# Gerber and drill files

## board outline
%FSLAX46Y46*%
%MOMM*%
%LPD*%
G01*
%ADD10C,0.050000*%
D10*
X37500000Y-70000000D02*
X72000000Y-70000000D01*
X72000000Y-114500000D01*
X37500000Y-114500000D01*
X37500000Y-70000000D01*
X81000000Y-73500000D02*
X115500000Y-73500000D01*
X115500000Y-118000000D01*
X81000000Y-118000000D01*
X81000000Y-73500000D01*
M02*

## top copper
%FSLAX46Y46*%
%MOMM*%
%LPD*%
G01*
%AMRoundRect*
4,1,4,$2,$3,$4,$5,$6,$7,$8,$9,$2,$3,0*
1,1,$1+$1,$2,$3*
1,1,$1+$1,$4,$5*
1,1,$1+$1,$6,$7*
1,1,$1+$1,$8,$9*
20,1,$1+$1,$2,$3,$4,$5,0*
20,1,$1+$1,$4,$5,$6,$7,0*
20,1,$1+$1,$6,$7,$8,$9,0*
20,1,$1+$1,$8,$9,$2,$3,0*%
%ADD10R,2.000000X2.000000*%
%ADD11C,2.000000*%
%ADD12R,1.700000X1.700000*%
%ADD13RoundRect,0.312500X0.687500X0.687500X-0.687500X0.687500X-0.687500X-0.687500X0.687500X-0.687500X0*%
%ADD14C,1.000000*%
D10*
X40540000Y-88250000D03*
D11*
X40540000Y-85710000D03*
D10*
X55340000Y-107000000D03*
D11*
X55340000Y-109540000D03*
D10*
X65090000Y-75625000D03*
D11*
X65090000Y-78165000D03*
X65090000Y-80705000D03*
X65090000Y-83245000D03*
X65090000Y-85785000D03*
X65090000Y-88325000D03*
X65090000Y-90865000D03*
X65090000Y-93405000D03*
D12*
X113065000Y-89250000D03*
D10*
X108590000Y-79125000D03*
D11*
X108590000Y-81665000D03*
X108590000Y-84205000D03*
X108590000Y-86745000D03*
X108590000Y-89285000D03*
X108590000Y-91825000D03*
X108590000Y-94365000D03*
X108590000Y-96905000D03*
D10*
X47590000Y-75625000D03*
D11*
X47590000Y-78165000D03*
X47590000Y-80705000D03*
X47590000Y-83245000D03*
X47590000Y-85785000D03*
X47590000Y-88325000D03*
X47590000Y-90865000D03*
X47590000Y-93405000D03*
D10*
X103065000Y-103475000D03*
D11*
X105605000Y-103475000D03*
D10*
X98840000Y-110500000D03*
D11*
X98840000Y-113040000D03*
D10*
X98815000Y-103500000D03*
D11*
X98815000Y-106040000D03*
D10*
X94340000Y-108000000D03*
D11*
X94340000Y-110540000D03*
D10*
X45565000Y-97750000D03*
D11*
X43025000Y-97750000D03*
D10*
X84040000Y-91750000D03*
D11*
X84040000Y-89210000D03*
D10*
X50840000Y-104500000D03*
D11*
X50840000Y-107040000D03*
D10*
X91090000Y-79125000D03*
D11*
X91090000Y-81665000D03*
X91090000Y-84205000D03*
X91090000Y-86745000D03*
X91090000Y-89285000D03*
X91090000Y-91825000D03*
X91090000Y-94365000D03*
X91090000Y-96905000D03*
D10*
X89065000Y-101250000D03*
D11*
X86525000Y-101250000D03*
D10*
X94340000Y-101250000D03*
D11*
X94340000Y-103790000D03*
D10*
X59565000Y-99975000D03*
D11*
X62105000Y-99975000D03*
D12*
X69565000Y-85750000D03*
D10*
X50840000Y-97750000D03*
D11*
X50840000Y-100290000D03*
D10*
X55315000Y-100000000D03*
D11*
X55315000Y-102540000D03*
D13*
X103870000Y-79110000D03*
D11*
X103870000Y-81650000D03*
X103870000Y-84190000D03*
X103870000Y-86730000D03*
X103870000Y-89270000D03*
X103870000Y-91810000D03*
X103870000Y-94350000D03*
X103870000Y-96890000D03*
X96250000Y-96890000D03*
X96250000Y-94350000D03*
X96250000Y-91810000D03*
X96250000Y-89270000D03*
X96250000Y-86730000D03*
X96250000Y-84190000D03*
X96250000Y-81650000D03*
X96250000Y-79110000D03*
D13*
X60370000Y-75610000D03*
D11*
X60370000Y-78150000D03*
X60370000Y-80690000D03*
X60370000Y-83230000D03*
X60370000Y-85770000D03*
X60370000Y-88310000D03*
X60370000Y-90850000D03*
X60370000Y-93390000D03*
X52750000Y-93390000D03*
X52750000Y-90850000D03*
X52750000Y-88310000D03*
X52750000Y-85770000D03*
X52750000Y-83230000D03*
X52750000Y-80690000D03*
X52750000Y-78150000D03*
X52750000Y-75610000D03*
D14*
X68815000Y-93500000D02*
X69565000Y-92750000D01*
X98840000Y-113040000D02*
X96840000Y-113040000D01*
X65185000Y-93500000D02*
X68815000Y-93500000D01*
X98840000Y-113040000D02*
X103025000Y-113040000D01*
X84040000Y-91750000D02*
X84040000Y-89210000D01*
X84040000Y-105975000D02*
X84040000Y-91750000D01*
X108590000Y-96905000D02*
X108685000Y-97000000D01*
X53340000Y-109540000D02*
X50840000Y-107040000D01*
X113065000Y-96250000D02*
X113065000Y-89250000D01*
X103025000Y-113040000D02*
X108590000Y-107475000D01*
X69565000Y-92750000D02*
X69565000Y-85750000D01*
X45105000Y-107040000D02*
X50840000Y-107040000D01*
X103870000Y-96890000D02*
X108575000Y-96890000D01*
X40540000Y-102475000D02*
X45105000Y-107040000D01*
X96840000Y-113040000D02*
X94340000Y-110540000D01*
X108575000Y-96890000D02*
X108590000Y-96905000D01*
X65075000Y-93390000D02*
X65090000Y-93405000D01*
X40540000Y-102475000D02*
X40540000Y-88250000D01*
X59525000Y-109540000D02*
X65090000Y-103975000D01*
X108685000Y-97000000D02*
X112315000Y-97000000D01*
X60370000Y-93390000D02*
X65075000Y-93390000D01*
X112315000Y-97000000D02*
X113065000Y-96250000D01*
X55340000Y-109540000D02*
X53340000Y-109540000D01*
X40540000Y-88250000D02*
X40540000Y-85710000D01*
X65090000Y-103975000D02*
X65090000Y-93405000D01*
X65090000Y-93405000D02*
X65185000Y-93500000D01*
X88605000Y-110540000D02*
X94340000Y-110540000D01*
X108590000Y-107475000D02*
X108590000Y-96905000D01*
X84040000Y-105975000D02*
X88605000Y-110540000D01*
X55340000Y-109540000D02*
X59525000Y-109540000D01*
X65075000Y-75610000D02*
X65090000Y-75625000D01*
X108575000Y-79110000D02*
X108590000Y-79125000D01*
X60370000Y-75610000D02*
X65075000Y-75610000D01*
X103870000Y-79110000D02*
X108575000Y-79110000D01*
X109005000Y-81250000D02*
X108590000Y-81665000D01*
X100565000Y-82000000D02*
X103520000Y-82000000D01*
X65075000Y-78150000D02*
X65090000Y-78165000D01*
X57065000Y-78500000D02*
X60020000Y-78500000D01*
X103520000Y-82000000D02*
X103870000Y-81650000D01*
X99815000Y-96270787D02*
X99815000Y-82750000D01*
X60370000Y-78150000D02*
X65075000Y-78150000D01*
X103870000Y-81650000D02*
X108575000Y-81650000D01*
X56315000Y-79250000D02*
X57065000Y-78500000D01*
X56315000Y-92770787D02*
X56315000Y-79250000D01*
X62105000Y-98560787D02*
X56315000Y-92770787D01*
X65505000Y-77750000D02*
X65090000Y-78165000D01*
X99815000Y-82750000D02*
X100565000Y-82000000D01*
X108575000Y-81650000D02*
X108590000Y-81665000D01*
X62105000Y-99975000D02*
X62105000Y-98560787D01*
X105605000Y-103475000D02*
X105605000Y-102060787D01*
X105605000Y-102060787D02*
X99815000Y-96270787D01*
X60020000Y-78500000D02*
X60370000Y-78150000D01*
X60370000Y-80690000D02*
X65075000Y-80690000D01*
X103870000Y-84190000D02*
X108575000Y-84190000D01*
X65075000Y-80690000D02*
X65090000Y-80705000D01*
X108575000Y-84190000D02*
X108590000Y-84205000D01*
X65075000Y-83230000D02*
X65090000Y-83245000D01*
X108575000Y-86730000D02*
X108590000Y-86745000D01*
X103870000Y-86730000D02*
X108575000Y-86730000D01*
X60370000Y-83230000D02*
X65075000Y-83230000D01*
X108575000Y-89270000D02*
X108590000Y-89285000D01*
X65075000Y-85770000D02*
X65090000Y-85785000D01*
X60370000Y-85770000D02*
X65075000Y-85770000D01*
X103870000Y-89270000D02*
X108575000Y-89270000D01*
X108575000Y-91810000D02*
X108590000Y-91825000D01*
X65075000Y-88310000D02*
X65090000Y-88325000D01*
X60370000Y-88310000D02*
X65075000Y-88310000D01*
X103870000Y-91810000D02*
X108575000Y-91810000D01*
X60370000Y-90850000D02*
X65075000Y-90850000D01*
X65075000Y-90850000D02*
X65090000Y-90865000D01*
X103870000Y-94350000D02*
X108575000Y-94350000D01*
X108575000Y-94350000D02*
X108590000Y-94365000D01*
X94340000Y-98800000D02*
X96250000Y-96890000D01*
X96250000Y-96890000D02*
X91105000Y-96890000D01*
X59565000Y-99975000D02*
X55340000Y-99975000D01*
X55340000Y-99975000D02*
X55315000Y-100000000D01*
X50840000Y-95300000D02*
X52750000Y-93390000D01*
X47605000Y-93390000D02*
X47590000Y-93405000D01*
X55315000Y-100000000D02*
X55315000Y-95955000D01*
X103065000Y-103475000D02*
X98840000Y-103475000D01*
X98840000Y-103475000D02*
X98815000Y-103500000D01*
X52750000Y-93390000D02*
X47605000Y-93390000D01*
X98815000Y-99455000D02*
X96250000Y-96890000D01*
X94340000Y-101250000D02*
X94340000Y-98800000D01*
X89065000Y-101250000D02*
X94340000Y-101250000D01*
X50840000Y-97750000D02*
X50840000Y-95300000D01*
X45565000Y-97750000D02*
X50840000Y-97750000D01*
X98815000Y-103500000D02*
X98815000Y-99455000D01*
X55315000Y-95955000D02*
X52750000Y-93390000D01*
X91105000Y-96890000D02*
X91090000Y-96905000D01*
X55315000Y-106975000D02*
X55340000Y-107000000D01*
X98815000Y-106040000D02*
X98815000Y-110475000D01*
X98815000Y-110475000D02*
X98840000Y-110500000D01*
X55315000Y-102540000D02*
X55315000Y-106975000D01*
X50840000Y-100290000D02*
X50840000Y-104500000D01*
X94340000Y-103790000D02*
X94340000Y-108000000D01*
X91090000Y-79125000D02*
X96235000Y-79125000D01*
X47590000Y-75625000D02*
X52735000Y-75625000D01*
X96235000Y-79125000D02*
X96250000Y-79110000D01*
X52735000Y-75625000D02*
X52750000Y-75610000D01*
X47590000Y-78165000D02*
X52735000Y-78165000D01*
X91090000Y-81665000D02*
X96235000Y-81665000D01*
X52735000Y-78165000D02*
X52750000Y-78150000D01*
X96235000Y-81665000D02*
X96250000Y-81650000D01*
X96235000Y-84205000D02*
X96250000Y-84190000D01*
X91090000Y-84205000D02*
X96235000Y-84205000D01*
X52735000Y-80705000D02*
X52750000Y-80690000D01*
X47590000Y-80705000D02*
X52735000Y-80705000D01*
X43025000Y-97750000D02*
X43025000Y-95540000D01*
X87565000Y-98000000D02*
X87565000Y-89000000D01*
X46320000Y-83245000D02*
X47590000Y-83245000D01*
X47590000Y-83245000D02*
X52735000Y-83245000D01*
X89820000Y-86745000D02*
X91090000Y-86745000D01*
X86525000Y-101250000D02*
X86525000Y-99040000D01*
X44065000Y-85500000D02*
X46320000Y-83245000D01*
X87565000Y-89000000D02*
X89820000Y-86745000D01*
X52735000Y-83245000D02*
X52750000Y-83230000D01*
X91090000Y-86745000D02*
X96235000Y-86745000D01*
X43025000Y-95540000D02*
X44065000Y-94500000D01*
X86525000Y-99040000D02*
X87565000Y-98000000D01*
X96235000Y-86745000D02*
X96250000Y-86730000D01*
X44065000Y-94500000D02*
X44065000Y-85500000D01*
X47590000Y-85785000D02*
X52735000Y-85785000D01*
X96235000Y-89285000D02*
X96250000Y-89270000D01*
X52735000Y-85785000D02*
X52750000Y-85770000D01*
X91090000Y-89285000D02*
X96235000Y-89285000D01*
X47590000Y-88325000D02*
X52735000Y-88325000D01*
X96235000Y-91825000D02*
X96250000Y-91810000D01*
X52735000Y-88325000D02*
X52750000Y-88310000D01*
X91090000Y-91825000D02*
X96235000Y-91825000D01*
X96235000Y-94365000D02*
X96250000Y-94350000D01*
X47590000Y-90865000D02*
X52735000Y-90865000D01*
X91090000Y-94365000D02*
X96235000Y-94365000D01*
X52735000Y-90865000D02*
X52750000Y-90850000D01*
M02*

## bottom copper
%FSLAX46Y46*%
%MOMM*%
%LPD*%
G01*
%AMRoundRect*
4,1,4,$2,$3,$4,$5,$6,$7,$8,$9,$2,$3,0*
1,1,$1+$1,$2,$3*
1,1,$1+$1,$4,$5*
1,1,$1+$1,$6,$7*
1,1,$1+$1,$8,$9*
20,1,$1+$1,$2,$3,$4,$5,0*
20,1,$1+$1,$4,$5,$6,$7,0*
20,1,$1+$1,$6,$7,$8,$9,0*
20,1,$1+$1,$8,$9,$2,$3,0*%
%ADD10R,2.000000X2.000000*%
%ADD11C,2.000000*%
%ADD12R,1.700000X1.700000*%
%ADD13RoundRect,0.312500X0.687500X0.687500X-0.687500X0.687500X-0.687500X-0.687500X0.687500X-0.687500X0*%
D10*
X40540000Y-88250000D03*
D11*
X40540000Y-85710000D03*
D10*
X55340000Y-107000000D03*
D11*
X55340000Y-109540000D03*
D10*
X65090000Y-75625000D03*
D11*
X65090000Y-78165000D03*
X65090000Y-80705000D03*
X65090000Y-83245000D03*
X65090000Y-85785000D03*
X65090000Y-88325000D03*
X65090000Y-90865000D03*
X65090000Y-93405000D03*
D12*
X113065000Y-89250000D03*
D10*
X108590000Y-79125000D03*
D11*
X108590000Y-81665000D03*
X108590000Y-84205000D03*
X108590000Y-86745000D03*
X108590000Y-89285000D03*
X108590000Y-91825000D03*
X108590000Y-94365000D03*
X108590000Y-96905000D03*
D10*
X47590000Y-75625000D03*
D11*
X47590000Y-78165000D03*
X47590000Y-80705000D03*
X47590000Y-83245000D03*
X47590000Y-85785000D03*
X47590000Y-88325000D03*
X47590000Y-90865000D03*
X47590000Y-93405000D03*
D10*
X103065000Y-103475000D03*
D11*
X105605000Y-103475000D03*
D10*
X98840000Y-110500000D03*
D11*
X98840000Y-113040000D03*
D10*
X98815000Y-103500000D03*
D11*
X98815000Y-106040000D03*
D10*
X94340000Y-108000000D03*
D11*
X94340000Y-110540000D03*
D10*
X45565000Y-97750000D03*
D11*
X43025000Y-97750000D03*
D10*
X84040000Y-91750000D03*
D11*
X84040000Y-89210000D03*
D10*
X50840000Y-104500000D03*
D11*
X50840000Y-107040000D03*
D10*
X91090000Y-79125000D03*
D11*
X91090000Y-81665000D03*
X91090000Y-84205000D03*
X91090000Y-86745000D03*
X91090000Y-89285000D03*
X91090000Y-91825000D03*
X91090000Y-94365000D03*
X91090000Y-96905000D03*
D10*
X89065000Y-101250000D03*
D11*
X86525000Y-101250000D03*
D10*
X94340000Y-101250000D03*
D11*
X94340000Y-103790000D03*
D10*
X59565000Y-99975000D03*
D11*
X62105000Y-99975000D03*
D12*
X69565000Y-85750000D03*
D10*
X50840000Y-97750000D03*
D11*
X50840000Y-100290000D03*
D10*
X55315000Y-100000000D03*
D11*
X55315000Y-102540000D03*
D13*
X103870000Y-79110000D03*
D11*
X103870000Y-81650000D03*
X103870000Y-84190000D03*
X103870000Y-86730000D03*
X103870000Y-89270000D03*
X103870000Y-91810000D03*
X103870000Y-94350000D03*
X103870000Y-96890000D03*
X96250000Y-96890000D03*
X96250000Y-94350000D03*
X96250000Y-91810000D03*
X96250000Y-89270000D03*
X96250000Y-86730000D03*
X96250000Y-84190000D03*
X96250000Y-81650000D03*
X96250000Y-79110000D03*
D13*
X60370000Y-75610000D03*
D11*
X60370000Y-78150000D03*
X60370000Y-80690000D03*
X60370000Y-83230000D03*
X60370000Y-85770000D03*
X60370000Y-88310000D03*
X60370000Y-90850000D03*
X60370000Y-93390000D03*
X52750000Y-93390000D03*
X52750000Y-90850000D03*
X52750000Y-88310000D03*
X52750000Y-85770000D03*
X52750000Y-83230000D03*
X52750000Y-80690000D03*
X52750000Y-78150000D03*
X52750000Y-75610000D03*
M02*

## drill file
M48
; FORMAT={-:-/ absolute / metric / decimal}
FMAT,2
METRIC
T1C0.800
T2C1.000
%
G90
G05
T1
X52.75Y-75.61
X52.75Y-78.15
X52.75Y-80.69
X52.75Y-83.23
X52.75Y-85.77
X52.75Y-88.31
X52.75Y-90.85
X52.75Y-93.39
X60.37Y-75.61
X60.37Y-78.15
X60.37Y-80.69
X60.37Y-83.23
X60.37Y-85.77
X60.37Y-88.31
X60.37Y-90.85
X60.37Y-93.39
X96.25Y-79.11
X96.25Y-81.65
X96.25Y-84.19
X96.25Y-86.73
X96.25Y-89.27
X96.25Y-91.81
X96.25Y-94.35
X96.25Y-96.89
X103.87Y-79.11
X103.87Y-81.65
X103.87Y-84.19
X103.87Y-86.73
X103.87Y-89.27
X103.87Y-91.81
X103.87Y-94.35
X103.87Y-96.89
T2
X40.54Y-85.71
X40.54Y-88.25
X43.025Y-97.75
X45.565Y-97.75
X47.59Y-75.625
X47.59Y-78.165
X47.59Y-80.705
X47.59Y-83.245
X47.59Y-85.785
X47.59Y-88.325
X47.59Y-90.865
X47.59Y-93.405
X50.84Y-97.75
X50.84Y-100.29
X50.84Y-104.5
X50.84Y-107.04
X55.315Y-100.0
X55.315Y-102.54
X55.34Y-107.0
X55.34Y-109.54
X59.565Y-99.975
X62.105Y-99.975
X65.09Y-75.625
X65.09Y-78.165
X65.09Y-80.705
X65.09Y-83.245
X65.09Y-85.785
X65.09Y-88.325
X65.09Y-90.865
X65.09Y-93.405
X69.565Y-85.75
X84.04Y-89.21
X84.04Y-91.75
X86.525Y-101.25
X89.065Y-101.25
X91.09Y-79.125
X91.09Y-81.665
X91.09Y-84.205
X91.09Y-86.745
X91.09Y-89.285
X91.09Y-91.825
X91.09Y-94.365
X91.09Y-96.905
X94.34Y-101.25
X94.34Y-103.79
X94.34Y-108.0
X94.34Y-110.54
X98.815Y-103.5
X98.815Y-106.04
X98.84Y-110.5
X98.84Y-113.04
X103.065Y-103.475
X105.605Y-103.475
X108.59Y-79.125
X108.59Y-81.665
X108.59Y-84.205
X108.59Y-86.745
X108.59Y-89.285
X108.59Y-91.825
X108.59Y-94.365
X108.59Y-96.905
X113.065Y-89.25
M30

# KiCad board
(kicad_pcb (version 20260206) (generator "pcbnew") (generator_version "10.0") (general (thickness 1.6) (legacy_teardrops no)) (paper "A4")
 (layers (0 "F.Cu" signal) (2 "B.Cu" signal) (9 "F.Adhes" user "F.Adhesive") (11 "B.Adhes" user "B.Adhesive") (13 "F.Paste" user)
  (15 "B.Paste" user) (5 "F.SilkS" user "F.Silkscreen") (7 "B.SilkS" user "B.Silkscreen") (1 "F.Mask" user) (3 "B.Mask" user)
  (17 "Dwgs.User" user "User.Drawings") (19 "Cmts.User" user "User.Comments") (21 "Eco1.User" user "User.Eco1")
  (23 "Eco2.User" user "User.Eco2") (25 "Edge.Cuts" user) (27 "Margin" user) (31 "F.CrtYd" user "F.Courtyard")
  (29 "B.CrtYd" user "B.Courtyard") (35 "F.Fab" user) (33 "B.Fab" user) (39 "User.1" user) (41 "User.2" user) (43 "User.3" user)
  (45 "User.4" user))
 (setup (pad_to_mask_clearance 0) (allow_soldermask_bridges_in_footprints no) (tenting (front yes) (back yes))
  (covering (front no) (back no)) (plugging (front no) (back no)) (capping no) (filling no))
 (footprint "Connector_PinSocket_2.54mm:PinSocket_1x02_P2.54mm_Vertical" (layer "F.Cu") (at 40.54 88.25 180)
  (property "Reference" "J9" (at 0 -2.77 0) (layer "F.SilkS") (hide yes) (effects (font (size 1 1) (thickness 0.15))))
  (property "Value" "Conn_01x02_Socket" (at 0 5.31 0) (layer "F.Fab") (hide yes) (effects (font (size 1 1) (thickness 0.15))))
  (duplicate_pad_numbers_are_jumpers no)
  (pad "1" thru_hole rect (at 0 0 180) (size 2 2) (drill 1) (layers "*.Cu" "*.Mask") (remove_unused_layers no) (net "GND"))
  (pad "2" thru_hole circle (at 0 2.54 180) (size 2 2) (drill 1) (layers "*.Cu" "*.Mask") (remove_unused_layers no) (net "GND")))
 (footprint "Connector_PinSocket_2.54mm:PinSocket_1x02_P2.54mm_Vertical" (layer "F.Cu") (at 55.34 107)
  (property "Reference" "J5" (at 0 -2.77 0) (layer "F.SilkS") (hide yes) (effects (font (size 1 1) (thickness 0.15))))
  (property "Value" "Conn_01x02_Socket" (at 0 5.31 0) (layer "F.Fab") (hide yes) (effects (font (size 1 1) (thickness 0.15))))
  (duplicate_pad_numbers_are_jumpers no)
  (pad "1" thru_hole rect (at 0 0) (size 2 2) (drill 1) (layers "*.Cu" "*.Mask") (remove_unused_layers no) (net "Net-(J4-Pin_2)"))
  (pad "2" thru_hole circle (at 0 2.54) (size 2 2) (drill 1) (layers "*.Cu" "*.Mask") (remove_unused_layers no) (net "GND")))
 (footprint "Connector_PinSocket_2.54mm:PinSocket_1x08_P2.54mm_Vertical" (layer "F.Cu") (at 65.09 75.625)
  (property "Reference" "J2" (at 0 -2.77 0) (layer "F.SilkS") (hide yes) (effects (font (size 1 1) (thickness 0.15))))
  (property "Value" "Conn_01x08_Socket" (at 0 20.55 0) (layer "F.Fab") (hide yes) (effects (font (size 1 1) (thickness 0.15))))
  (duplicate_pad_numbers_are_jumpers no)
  (pad "1" thru_hole rect (at 0 0) (size 2 2) (drill 1) (layers "*.Cu" "*.Mask") (remove_unused_layers no) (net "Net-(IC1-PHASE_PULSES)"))
  (pad "2" thru_hole circle (at 0 2.54) (size 2 2) (drill 1) (layers "*.Cu" "*.Mask") (remove_unused_layers no) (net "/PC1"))
  (pad "3" thru_hole circle (at 0 5.08) (size 2 2) (drill 1) (layers "*.Cu" "*.Mask") (remove_unused_layers no)
   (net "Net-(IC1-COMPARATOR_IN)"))
  (pad "4" thru_hole circle (at 0 7.62) (size 2 2) (drill 1) (layers "*.Cu" "*.Mask") (remove_unused_layers no) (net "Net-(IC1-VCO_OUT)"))
  (pad "5" thru_hole circle (at 0 10.16) (size 2 2) (drill 1) (layers "*.Cu" "*.Mask") (remove_unused_layers no) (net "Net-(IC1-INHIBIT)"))
  (pad "6" thru_hole circle (at 0 12.7) (size 2 2) (drill 1) (layers "*.Cu" "*.Mask") (remove_unused_layers no) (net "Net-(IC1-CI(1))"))
  (pad "7" thru_hole circle (at 0 15.24) (size 2 2) (drill 1) (layers "*.Cu" "*.Mask") (remove_unused_layers no) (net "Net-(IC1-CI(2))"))
  (pad "8" thru_hole circle (at 0 17.78) (size 2 2) (drill 1) (layers "*.Cu" "*.Mask") (remove_unused_layers no) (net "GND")))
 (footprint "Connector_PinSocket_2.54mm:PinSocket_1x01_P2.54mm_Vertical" (layer "F.Cu") (at 113.065 89.25)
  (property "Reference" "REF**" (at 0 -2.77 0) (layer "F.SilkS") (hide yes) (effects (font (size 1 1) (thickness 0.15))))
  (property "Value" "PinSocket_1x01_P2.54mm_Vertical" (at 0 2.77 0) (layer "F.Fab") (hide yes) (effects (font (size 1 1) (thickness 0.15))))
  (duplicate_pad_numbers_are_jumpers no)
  (pad "1" thru_hole rect (at 0 0) (size 1.7 1.7) (drill 1) (layers "*.Cu" "*.Mask") (remove_unused_layers no) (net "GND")))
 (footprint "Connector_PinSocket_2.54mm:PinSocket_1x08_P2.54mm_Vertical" (layer "F.Cu") (at 108.59 79.125)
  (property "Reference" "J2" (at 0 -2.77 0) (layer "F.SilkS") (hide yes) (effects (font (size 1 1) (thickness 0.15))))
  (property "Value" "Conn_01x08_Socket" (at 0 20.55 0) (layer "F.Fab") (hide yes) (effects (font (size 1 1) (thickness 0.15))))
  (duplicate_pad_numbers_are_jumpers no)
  (pad "1" thru_hole rect (at 0 0) (size 2 2) (drill 1) (layers "*.Cu" "*.Mask") (remove_unused_layers no) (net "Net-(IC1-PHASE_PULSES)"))
  (pad "2" thru_hole circle (at 0 2.54) (size 2 2) (drill 1) (layers "*.Cu" "*.Mask") (remove_unused_layers no) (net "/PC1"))
  (pad "3" thru_hole circle (at 0 5.08) (size 2 2) (drill 1) (layers "*.Cu" "*.Mask") (remove_unused_layers no)
   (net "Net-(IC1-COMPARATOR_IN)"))
  (pad "4" thru_hole circle (at 0 7.62) (size 2 2) (drill 1) (layers "*.Cu" "*.Mask") (remove_unused_layers no) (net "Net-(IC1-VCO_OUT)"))
  (pad "5" thru_hole circle (at 0 10.16) (size 2 2) (drill 1) (layers "*.Cu" "*.Mask") (remove_unused_layers no) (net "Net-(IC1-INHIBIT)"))
  (pad "6" thru_hole circle (at 0 12.7) (size 2 2) (drill 1) (layers "*.Cu" "*.Mask") (remove_unused_layers no) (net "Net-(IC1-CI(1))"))
  (pad "7" thru_hole circle (at 0 15.24) (size 2 2) (drill 1) (layers "*.Cu" "*.Mask") (remove_unused_layers no) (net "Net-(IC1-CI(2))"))
  (pad "8" thru_hole circle (at 0 17.78) (size 2 2) (drill 1) (layers "*.Cu" "*.Mask") (remove_unused_layers no) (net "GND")))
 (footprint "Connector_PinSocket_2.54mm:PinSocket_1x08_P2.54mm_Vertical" (layer "F.Cu") (at 47.59 75.625)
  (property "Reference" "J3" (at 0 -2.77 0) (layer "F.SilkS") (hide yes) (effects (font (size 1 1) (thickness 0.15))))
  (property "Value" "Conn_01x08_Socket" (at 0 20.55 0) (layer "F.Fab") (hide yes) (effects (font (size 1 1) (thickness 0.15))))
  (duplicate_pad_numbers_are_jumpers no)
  (pad "1" thru_hole rect (at 0 0) (size 2 2) (drill 1) (layers "*.Cu" "*.Mask") (remove_unused_layers no) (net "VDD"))
  (pad "2" thru_hole circle (at 0 2.54) (size 2 2) (drill 1) (layers "*.Cu" "*.Mask") (remove_unused_layers no) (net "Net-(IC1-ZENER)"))
  (pad "3" thru_hole circle (at 0 5.08) (size 2 2) (drill 1) (layers "*.Cu" "*.Mask") (remove_unused_layers no) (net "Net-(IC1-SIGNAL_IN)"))
  (pad "4" thru_hole circle (at 0 7.62) (size 2 2) (drill 1) (layers "*.Cu" "*.Mask") (remove_unused_layers no) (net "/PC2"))
  (pad "5" thru_hole circle (at 0 10.16) (size 2 2) (drill 1) (layers "*.Cu" "*.Mask") (remove_unused_layers no) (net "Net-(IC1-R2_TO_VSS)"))
  (pad "6" thru_hole circle (at 0 12.7) (size 2 2) (drill 1) (layers "*.Cu" "*.Mask") (remove_unused_layers no) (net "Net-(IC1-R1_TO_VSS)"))
  (pad "7" thru_hole circle (at 0 15.24) (size 2 2) (drill 1) (layers "*.Cu" "*.Mask") (remove_unused_layers no)
   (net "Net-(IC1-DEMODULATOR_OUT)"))
  (pad "8" thru_hole circle (at 0 17.78) (size 2 2) (drill 1) (layers "*.Cu" "*.Mask") (remove_unused_layers no) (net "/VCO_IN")))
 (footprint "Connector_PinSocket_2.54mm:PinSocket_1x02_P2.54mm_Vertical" (layer "F.Cu") (at 103.065 103.475 90)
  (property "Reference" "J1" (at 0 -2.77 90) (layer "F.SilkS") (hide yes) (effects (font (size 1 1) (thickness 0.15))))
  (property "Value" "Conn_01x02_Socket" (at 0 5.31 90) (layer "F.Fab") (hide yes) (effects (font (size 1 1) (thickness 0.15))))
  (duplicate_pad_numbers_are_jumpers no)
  (pad "1" thru_hole rect (at 0 0 90) (size 2 2) (drill 1) (layers "*.Cu" "*.Mask") (remove_unused_layers no) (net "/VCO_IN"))
  (pad "2" thru_hole circle (at 0 2.54 90) (size 2 2) (drill 1) (layers "*.Cu" "*.Mask") (remove_unused_layers no) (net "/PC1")))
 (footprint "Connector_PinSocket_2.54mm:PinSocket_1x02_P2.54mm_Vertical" (layer "F.Cu") (at 98.84 110.5)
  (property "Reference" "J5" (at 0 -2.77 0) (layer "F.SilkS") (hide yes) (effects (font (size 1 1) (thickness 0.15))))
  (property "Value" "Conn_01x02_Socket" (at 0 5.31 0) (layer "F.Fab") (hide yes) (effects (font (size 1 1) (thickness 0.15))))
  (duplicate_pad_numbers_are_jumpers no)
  (pad "1" thru_hole rect (at 0 0) (size 2 2) (drill 1) (layers "*.Cu" "*.Mask") (remove_unused_layers no) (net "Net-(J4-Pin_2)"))
  (pad "2" thru_hole circle (at 0 2.54) (size 2 2) (drill 1) (layers "*.Cu" "*.Mask") (remove_unused_layers no) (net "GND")))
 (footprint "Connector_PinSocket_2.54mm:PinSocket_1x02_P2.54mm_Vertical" (layer "F.Cu") (at 98.815 103.5)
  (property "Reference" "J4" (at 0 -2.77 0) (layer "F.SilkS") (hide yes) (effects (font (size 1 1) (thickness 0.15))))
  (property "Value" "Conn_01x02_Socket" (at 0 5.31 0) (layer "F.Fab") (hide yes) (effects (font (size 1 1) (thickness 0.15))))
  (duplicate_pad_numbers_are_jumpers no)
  (pad "1" thru_hole rect (at 0 0) (size 2 2) (drill 1) (layers "*.Cu" "*.Mask") (remove_unused_layers no) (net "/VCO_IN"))
  (pad "2" thru_hole circle (at 0 2.54) (size 2 2) (drill 1) (layers "*.Cu" "*.Mask") (remove_unused_layers no) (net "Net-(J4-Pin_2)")))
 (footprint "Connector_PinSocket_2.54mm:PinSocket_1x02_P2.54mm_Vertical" (layer "F.Cu") (at 94.34 108)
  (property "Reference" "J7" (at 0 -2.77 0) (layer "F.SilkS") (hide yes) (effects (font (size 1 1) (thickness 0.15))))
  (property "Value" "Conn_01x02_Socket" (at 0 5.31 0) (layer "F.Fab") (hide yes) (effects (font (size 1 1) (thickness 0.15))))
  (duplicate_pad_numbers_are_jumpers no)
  (pad "1" thru_hole rect (at 0 0) (size 2 2) (drill 1) (layers "*.Cu" "*.Mask") (remove_unused_layers no) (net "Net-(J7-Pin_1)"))
  (pad "2" thru_hole circle (at 0 2.54) (size 2 2) (drill 1) (layers "*.Cu" "*.Mask") (remove_unused_layers no) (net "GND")))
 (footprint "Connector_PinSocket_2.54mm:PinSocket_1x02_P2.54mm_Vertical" (layer "F.Cu") (at 45.565 97.75 -90)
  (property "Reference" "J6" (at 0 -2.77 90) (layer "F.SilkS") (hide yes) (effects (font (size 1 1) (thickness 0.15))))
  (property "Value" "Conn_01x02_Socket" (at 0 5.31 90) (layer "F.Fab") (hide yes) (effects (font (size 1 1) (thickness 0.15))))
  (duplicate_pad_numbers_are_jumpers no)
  (pad "1" thru_hole rect (at 0 0 270) (size 2 2) (drill 1) (layers "*.Cu" "*.Mask") (remove_unused_layers no) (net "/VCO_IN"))
  (pad "2" thru_hole circle (at 0 2.54 270) (size 2 2) (drill 1) (layers "*.Cu" "*.Mask") (remove_unused_layers no) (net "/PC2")))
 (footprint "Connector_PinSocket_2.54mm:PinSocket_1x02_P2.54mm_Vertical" (layer "F.Cu") (at 84.04 91.75 180)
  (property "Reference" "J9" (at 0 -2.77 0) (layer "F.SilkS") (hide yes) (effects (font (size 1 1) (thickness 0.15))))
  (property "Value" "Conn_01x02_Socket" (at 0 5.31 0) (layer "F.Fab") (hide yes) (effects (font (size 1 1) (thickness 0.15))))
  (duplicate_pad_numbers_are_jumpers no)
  (pad "1" thru_hole rect (at 0 0 180) (size 2 2) (drill 1) (layers "*.Cu" "*.Mask") (remove_unused_layers no) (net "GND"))
  (pad "2" thru_hole circle (at 0 2.54 180) (size 2 2) (drill 1) (layers "*.Cu" "*.Mask") (remove_unused_layers no) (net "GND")))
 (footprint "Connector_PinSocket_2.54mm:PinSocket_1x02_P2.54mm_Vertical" (layer "F.Cu") (at 50.84 104.5)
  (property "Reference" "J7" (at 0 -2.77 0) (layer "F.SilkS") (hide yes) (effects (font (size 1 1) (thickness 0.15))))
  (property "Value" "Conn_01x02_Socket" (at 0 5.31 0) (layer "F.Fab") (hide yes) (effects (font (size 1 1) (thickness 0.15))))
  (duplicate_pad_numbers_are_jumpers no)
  (pad "1" thru_hole rect (at 0 0) (size 2 2) (drill 1) (layers "*.Cu" "*.Mask") (remove_unused_layers no) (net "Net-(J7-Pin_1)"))
  (pad "2" thru_hole circle (at 0 2.54) (size 2 2) (drill 1) (layers "*.Cu" "*.Mask") (remove_unused_layers no) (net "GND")))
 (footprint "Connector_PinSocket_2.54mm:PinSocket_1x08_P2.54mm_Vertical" (layer "F.Cu") (at 91.09 79.125)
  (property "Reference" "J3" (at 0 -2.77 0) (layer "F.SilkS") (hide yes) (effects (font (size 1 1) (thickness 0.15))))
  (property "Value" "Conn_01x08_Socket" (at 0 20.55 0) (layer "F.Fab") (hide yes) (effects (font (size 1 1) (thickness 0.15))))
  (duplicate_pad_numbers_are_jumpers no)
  (pad "1" thru_hole rect (at 0 0) (size 2 2) (drill 1) (layers "*.Cu" "*.Mask") (remove_unused_layers no) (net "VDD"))
  (pad "2" thru_hole circle (at 0 2.54) (size 2 2) (drill 1) (layers "*.Cu" "*.Mask") (remove_unused_layers no) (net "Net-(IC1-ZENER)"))
  (pad "3" thru_hole circle (at 0 5.08) (size 2 2) (drill 1) (layers "*.Cu" "*.Mask") (remove_unused_layers no) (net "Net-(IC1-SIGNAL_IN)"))
  (pad "4" thru_hole circle (at 0 7.62) (size 2 2) (drill 1) (layers "*.Cu" "*.Mask") (remove_unused_layers no) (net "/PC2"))
  (pad "5" thru_hole circle (at 0 10.16) (size 2 2) (drill 1) (layers "*.Cu" "*.Mask") (remove_unused_layers no) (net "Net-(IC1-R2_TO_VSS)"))
  (pad "6" thru_hole circle (at 0 12.7) (size 2 2) (drill 1) (layers "*.Cu" "*.Mask") (remove_unused_layers no) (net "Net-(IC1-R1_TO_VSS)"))
  (pad "7" thru_hole circle (at 0 15.24) (size 2 2) (drill 1) (layers "*.Cu" "*.Mask") (remove_unused_layers no)
   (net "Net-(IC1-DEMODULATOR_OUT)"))
  (pad "8" thru_hole circle (at 0 17.78) (size 2 2) (drill 1) (layers "*.Cu" "*.Mask") (remove_unused_layers no) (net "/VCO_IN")))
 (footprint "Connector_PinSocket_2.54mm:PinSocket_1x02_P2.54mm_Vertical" (layer "F.Cu") (at 89.065 101.25 -90)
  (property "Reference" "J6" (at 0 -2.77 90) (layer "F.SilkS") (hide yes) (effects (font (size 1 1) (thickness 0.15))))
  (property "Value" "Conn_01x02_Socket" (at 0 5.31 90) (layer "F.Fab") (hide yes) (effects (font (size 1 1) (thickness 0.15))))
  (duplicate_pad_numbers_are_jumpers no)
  (pad "1" thru_hole rect (at 0 0 270) (size 2 2) (drill 1) (layers "*.Cu" "*.Mask") (remove_unused_layers no) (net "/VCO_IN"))
  (pad "2" thru_hole circle (at 0 2.54 270) (size 2 2) (drill 1) (layers "*.Cu" "*.Mask") (remove_unused_layers no) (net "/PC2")))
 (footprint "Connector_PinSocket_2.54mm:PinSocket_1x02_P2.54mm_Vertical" (layer "F.Cu") (at 94.34 101.25)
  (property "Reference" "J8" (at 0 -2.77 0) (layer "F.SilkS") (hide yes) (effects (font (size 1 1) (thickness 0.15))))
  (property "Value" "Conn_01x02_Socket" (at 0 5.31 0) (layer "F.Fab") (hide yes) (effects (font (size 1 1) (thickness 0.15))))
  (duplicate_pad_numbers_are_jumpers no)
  (pad "1" thru_hole rect (at 0 0) (size 2 2) (drill 1) (layers "*.Cu" "*.Mask") (remove_unused_layers no) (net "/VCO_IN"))
  (pad "2" thru_hole circle (at 0 2.54) (size 2 2) (drill 1) (layers "*.Cu" "*.Mask") (remove_unused_layers no) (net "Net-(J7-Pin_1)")))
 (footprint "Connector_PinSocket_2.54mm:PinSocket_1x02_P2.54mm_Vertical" (layer "F.Cu") (at 59.565 99.975 90)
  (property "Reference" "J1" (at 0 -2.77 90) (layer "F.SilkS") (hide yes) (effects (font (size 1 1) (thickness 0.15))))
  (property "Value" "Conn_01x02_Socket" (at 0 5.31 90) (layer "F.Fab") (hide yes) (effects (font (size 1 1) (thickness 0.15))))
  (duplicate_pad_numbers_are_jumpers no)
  (pad "1" thru_hole rect (at 0 0 90) (size 2 2) (drill 1) (layers "*.Cu" "*.Mask") (remove_unused_layers no) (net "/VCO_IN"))
  (pad "2" thru_hole circle (at 0 2.54 90) (size 2 2) (drill 1) (layers "*.Cu" "*.Mask") (remove_unused_layers no) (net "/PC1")))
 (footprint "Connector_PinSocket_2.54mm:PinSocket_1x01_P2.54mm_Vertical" (layer "F.Cu") (at 69.565 85.75)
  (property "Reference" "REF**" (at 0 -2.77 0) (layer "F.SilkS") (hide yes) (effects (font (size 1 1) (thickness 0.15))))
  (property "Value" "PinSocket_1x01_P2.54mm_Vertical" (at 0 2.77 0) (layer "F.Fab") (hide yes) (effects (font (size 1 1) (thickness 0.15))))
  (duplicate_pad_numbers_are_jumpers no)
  (pad "1" thru_hole rect (at 0 0) (size 1.7 1.7) (drill 1) (layers "*.Cu" "*.Mask") (remove_unused_layers no) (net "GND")))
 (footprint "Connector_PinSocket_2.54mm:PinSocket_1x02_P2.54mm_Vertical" (layer "F.Cu") (at 50.84 97.75)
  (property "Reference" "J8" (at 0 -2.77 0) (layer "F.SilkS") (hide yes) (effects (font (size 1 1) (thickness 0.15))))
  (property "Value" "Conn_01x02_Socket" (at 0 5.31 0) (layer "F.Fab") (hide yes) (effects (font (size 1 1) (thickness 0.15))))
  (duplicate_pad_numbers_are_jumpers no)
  (pad "1" thru_hole rect (at 0 0) (size 2 2) (drill 1) (layers "*.Cu" "*.Mask") (remove_unused_layers no) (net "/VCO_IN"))
  (pad "2" thru_hole circle (at 0 2.54) (size 2 2) (drill 1) (layers "*.Cu" "*.Mask") (remove_unused_layers no) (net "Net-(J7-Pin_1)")))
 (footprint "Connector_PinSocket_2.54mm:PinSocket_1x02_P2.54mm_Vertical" (layer "F.Cu") (at 55.315 100)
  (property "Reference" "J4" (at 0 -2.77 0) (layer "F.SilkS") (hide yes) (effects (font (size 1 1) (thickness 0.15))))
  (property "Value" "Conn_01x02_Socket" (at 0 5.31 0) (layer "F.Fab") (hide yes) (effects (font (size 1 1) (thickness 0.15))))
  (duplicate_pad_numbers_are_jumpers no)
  (pad "1" thru_hole rect (at 0 0) (size 2 2) (drill 1) (layers "*.Cu" "*.Mask") (remove_unused_layers no) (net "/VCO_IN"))
  (pad "2" thru_hole circle (at 0 2.54) (size 2 2) (drill 1) (layers "*.Cu" "*.Mask") (remove_unused_layers no) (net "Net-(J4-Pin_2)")))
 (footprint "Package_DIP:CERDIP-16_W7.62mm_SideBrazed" (layer "B.Cu") (at 103.87 79.11 180)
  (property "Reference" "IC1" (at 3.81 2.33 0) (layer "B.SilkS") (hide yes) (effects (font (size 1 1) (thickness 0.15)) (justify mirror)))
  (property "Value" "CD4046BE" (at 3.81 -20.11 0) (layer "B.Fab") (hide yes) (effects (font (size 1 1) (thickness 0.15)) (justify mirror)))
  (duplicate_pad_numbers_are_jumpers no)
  (pad "1" thru_hole roundrect (at 0 0 180) (size 2 2) (drill 0.8) (layers "*.Cu" "*.Mask") (remove_unused_layers no)
   (roundrect_rratio 0.15625) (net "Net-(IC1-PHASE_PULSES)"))
  (pad "2" thru_hole circle (at 0 -2.54 180) (size 2 2) (drill 0.8) (layers "*.Cu" "*.Mask") (remove_unused_layers no) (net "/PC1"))
  (pad "3" thru_hole circle (at 0 -5.08 180) (size 2 2) (drill 0.8) (layers "*.Cu" "*.Mask") (remove_unused_layers no)
   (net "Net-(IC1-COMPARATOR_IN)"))
  (pad "4" thru_hole circle (at 0 -7.62 180) (size 2 2) (drill 0.8) (layers "*.Cu" "*.Mask") (remove_unused_layers no)
   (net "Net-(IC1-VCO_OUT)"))
  (pad "5" thru_hole circle (at 0 -10.16 180) (size 2 2) (drill 0.8) (layers "*.Cu" "*.Mask") (remove_unused_layers no)
   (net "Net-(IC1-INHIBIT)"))
  (pad "6" thru_hole circle (at 0 -12.7 180) (size 2 2) (drill 0.8) (layers "*.Cu" "*.Mask") (remove_unused_layers no)
   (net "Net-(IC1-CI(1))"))
  (pad "7" thru_hole circle (at 0 -15.24 180) (size 2 2) (drill 0.8) (layers "*.Cu" "*.Mask") (remove_unused_layers no)
   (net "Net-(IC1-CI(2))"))
  (pad "8" thru_hole circle (at 0 -17.78 180) (size 2 2) (drill 0.8) (layers "*.Cu" "*.Mask") (remove_unused_layers no) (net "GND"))
  (pad "9" thru_hole circle (at 7.62 -17.78 180) (size 2 2) (drill 0.8) (layers "*.Cu" "*.Mask") (remove_unused_layers no) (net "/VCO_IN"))
  (pad "10" thru_hole circle (at 7.62 -15.24 180) (size 2 2) (drill 0.8) (layers "*.Cu" "*.Mask") (remove_unused_layers no)
   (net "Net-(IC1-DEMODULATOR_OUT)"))
  (pad "11" thru_hole circle (at 7.62 -12.7 180) (size 2 2) (drill 0.8) (layers "*.Cu" "*.Mask") (remove_unused_layers no)
   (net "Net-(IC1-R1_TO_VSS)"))
  (pad "12" thru_hole circle (at 7.62 -10.16 180) (size 2 2) (drill 0.8) (layers "*.Cu" "*.Mask") (remove_unused_layers no)
   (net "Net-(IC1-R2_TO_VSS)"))
  (pad "13" thru_hole circle (at 7.62 -7.62 180) (size 2 2) (drill 0.8) (layers "*.Cu" "*.Mask") (remove_unused_layers no) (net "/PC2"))
  (pad "14" thru_hole circle (at 7.62 -5.08 180) (size 2 2) (drill 0.8) (layers "*.Cu" "*.Mask") (remove_unused_layers no)
   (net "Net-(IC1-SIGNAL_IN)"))
  (pad "15" thru_hole circle (at 7.62 -2.54 180) (size 2 2) (drill 0.8) (layers "*.Cu" "*.Mask") (remove_unused_layers no)
   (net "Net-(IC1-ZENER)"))
  (pad "16" thru_hole circle (at 7.62 0 180) (size 2 2) (drill 0.8) (layers "*.Cu" "*.Mask") (remove_unused_layers no) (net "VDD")))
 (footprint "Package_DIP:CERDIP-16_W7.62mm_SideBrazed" (layer "B.Cu") (at 60.37 75.61 180)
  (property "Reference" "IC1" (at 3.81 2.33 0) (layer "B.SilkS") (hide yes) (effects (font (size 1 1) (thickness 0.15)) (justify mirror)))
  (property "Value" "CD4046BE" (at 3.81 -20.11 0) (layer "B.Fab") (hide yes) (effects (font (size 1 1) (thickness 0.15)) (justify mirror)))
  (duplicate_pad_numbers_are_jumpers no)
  (pad "1" thru_hole roundrect (at 0 0 180) (size 2 2) (drill 0.8) (layers "*.Cu" "*.Mask") (remove_unused_layers no)
   (roundrect_rratio 0.15625) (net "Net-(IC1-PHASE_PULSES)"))
  (pad "2" thru_hole circle (at 0 -2.54 180) (size 2 2) (drill 0.8) (layers "*.Cu" "*.Mask") (remove_unused_layers no) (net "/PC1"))
  (pad "3" thru_hole circle (at 0 -5.08 180) (size 2 2) (drill 0.8) (layers "*.Cu" "*.Mask") (remove_unused_layers no)
   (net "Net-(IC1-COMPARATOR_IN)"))
  (pad "4" thru_hole circle (at 0 -7.62 180) (size 2 2) (drill 0.8) (layers "*.Cu" "*.Mask") (remove_unused_layers no)
   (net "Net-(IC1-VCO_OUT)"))
  (pad "5" thru_hole circle (at 0 -10.16 180) (size 2 2) (drill 0.8) (layers "*.Cu" "*.Mask") (remove_unused_layers no)
   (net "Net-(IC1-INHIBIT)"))
  (pad "6" thru_hole circle (at 0 -12.7 180) (size 2 2) (drill 0.8) (layers "*.Cu" "*.Mask") (remove_unused_layers no)
   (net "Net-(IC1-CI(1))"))
  (pad "7" thru_hole circle (at 0 -15.24 180) (size 2 2) (drill 0.8) (layers "*.Cu" "*.Mask") (remove_unused_layers no)
   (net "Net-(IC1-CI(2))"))
  (pad "8" thru_hole circle (at 0 -17.78 180) (size 2 2) (drill 0.8) (layers "*.Cu" "*.Mask") (remove_unused_layers no) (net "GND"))
  (pad "9" thru_hole circle (at 7.62 -17.78 180) (size 2 2) (drill 0.8) (layers "*.Cu" "*.Mask") (remove_unused_layers no) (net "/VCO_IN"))
  (pad "10" thru_hole circle (at 7.62 -15.24 180) (size 2 2) (drill 0.8) (layers "*.Cu" "*.Mask") (remove_unused_layers no)
   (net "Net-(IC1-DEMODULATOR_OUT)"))
  (pad "11" thru_hole circle (at 7.62 -12.7 180) (size 2 2) (drill 0.8) (layers "*.Cu" "*.Mask") (remove_unused_layers no)
   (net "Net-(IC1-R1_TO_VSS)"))
  (pad "12" thru_hole circle (at 7.62 -10.16 180) (size 2 2) (drill 0.8) (layers "*.Cu" "*.Mask") (remove_unused_layers no)
   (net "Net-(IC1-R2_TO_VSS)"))
  (pad "13" thru_hole circle (at 7.62 -7.62 180) (size 2 2) (drill 0.8) (layers "*.Cu" "*.Mask") (remove_unused_layers no) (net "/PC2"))
  (pad "14" thru_hole circle (at 7.62 -5.08 180) (size 2 2) (drill 0.8) (layers "*.Cu" "*.Mask") (remove_unused_layers no)
   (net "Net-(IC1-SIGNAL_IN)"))
  (pad "15" thru_hole circle (at 7.62 -2.54 180) (size 2 2) (drill 0.8) (layers "*.Cu" "*.Mask") (remove_unused_layers no)
   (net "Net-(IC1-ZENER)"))
  (pad "16" thru_hole circle (at 7.62 0 180) (size 2 2) (drill 0.8) (layers "*.Cu" "*.Mask") (remove_unused_layers no) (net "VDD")))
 (gr_rect (start 37.5 70) (end 72 114.5) (stroke (width 0.05) (type default)) (fill no) (layer "Edge.Cuts"))
 (gr_rect (start 81 73.5) (end 115.5 118) (stroke (width 0.05) (type default)) (fill no) (layer "Edge.Cuts"))
 (segment (start 68.815 93.5) (end 69.565 92.75) (width 1) (layer "F.Cu") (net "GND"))
 (segment (start 98.84 113.04) (end 96.84 113.04) (width 1) (layer "F.Cu") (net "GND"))
 (segment (start 65.185 93.5) (end 68.815 93.5) (width 1) (layer "F.Cu") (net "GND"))
 (segment (start 98.84 113.04) (end 103.025 113.04) (width 1) (layer "F.Cu") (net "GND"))
 (segment (start 84.04 91.75) (end 84.04 89.21) (width 1) (layer "F.Cu") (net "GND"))
 (segment (start 84.04 105.975) (end 84.04 91.75) (width 1) (layer "F.Cu") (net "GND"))
 (segment (start 108.59 96.905) (end 108.685 97) (width 1) (layer "F.Cu") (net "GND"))
 (segment (start 53.34 109.54) (end 50.84 107.04) (width 1) (layer "F.Cu") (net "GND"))
 (segment (start 113.065 96.25) (end 113.065 89.25) (width 1) (layer "F.Cu") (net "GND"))
 (segment (start 103.025 113.04) (end 108.59 107.475) (width 1) (layer "F.Cu") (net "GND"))
 (segment (start 69.565 92.75) (end 69.565 85.75) (width 1) (layer "F.Cu") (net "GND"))
 (segment (start 45.105 107.04) (end 50.84 107.04) (width 1) (layer "F.Cu") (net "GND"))
 (segment (start 103.87 96.89) (end 108.575 96.89) (width 1) (layer "F.Cu") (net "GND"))
 (segment (start 40.54 102.475) (end 45.105 107.04) (width 1) (layer "F.Cu") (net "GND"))
 (segment (start 96.84 113.04) (end 94.34 110.54) (width 1) (layer "F.Cu") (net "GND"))
 (segment (start 108.575 96.89) (end 108.59 96.905) (width 1) (layer "F.Cu") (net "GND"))
 (segment (start 65.075 93.39) (end 65.09 93.405) (width 1) (layer "F.Cu") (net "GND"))
 (segment (start 40.54 102.475) (end 40.54 88.25) (width 1) (layer "F.Cu") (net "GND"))
 (segment (start 59.525 109.54) (end 65.09 103.975) (width 1) (layer "F.Cu") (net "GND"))
 (segment (start 108.685 97) (end 112.315 97) (width 1) (layer "F.Cu") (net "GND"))
 (segment (start 60.37 93.39) (end 65.075 93.39) (width 1) (layer "F.Cu") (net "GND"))
 (segment (start 112.315 97) (end 113.065 96.25) (width 1) (layer "F.Cu") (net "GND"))
 (segment (start 55.34 109.54) (end 53.34 109.54) (width 1) (layer "F.Cu") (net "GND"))
 (segment (start 40.54 88.25) (end 40.54 85.71) (width 1) (layer "F.Cu") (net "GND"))
 (segment (start 65.09 103.975) (end 65.09 93.405) (width 1) (layer "F.Cu") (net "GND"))
 (segment (start 65.09 93.405) (end 65.185 93.5) (width 1) (layer "F.Cu") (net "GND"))
 (segment (start 88.605 110.54) (end 94.34 110.54) (width 1) (layer "F.Cu") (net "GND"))
 (segment (start 108.59 107.475) (end 108.59 96.905) (width 1) (layer "F.Cu") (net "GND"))
 (segment (start 84.04 105.975) (end 88.605 110.54) (width 1) (layer "F.Cu") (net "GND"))
 (segment (start 55.34 109.54) (end 59.525 109.54) (width 1) (layer "F.Cu") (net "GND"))
 (segment (start 65.075 75.61) (end 65.09 75.625) (width 1) (layer "F.Cu") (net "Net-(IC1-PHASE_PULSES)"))
 (segment (start 108.575 79.11) (end 108.59 79.125) (width 1) (layer "F.Cu") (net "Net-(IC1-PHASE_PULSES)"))
 (segment (start 60.37 75.61) (end 65.075 75.61) (width 1) (layer "F.Cu") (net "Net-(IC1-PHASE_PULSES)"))
 (segment (start 103.87 79.11) (end 108.575 79.11) (width 1) (layer "F.Cu") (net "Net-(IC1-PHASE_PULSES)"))
 (segment (start 109.005 81.25) (end 108.59 81.665) (width 1) (layer "F.Cu") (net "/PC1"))
 (segment (start 100.565 82) (end 103.52 82) (width 1) (layer "F.Cu") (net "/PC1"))
 (segment (start 65.075 78.15) (end 65.09 78.165) (width 1) (layer "F.Cu") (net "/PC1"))
 (segment (start 57.065 78.5) (end 60.02 78.5) (width 1) (layer "F.Cu") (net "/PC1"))
 (segment (start 103.52 82) (end 103.87 81.65) (width 1) (layer "F.Cu") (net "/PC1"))
 (segment (start 99.815 96.270787) (end 99.815 82.75) (width 1) (layer "F.Cu") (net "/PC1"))
 (segment (start 60.37 78.15) (end 65.075 78.15) (width 1) (layer "F.Cu") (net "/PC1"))
 (segment (start 103.87 81.65) (end 108.575 81.65) (width 1) (layer "F.Cu") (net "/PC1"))
 (segment (start 56.315 79.25) (end 57.065 78.5) (width 1) (layer "F.Cu") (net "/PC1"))
 (segment (start 56.315 92.770787) (end 56.315 79.25) (width 1) (layer "F.Cu") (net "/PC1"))
 (segment (start 62.105 98.560787) (end 56.315 92.770787) (width 1) (layer "F.Cu") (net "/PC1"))
 (segment (start 65.505 77.75) (end 65.09 78.165) (width 1) (layer "F.Cu") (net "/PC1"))
 (segment (start 99.815 82.75) (end 100.565 82) (width 1) (layer "F.Cu") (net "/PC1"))
 (segment (start 108.575 81.65) (end 108.59 81.665) (width 1) (layer "F.Cu") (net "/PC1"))
 (segment (start 62.105 99.975) (end 62.105 98.560787) (width 1) (layer "F.Cu") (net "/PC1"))
 (segment (start 105.605 103.475) (end 105.605 102.060787) (width 1) (layer "F.Cu") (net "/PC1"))
 (segment (start 105.605 102.060787) (end 99.815 96.270787) (width 1) (layer "F.Cu") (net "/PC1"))
 (segment (start 60.02 78.5) (end 60.37 78.15) (width 1) (layer "F.Cu") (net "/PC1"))
 (segment (start 60.37 80.69) (end 65.075 80.69) (width 1) (layer "F.Cu") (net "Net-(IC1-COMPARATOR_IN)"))
 (segment (start 103.87 84.19) (end 108.575 84.19) (width 1) (layer "F.Cu") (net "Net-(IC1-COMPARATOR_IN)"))
 (segment (start 65.075 80.69) (end 65.09 80.705) (width 1) (layer "F.Cu") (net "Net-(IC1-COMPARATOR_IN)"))
 (segment (start 108.575 84.19) (end 108.59 84.205) (width 1) (layer "F.Cu") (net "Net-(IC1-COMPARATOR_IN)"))
 (segment (start 65.075 83.23) (end 65.09 83.245) (width 1) (layer "F.Cu") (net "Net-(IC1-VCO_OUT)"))
 (segment (start 108.575 86.73) (end 108.59 86.745) (width 1) (layer "F.Cu") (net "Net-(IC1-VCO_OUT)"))
 (segment (start 103.87 86.73) (end 108.575 86.73) (width 1) (layer "F.Cu") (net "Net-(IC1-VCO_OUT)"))
 (segment (start 60.37 83.23) (end 65.075 83.23) (width 1) (layer "F.Cu") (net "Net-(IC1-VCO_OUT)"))
 (segment (start 108.575 89.27) (end 108.59 89.285) (width 1) (layer "F.Cu") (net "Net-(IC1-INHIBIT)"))
 (segment (start 65.075 85.77) (end 65.09 85.785) (width 1) (layer "F.Cu") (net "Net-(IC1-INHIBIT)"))
 (segment (start 60.37 85.77) (end 65.075 85.77) (width 1) (layer "F.Cu") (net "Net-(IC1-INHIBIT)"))
 (segment (start 103.87 89.27) (end 108.575 89.27) (width 1) (layer "F.Cu") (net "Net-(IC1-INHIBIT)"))
 (segment (start 108.575 91.81) (end 108.59 91.825) (width 1) (layer "F.Cu") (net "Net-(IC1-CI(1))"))
 (segment (start 65.075 88.31) (end 65.09 88.325) (width 1) (layer "F.Cu") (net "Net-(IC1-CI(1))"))
 (segment (start 60.37 88.31) (end 65.075 88.31) (width 1) (layer "F.Cu") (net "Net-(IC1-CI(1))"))
 (segment (start 103.87 91.81) (end 108.575 91.81) (width 1) (layer "F.Cu") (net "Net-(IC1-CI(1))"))
 (segment (start 60.37 90.85) (end 65.075 90.85) (width 1) (layer "F.Cu") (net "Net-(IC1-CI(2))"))
 (segment (start 65.075 90.85) (end 65.09 90.865) (width 1) (layer "F.Cu") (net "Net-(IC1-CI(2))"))
 (segment (start 103.87 94.35) (end 108.575 94.35) (width 1) (layer "F.Cu") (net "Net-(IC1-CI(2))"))
 (segment (start 108.575 94.35) (end 108.59 94.365) (width 1) (layer "F.Cu") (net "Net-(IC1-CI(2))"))
 (segment (start 94.34 98.8) (end 96.25 96.89) (width 1) (layer "F.Cu") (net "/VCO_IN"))
 (segment (start 96.25 96.89) (end 91.105 96.89) (width 1) (layer "F.Cu") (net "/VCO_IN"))
 (segment (start 59.565 99.975) (end 55.34 99.975) (width 1) (layer "F.Cu") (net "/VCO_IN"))
 (segment (start 55.34 99.975) (end 55.315 100) (width 1) (layer "F.Cu") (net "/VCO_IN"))
 (segment (start 50.84 95.3) (end 52.75 93.39) (width 1) (layer "F.Cu") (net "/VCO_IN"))
 (segment (start 47.605 93.39) (end 47.59 93.405) (width 1) (layer "F.Cu") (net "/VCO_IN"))
 (segment (start 55.315 100) (end 55.315 95.955) (width 1) (layer "F.Cu") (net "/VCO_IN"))
 (segment (start 103.065 103.475) (end 98.84 103.475) (width 1) (layer "F.Cu") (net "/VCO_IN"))
 (segment (start 98.84 103.475) (end 98.815 103.5) (width 1) (layer "F.Cu") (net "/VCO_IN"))
 (segment (start 52.75 93.39) (end 47.605 93.39) (width 1) (layer "F.Cu") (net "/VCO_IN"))
 (segment (start 98.815 99.455) (end 96.25 96.89) (width 1) (layer "F.Cu") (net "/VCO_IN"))
 (segment (start 94.34 101.25) (end 94.34 98.8) (width 1) (layer "F.Cu") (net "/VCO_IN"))
 (segment (start 89.065 101.25) (end 94.34 101.25) (width 1) (layer "F.Cu") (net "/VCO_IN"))
 (segment (start 50.84 97.75) (end 50.84 95.3) (width 1) (layer "F.Cu") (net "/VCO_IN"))
 (segment (start 45.565 97.75) (end 50.84 97.75) (width 1) (layer "F.Cu") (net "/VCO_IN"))
 (segment (start 98.815 103.5) (end 98.815 99.455) (width 1) (layer "F.Cu") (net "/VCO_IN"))
 (segment (start 55.315 95.955) (end 52.75 93.39) (width 1) (layer "F.Cu") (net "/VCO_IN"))
 (segment (start 91.105 96.89) (end 91.09 96.905) (width 1) (layer "F.Cu") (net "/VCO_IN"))
 (segment (start 55.315 106.975) (end 55.34 107) (width 1) (layer "F.Cu") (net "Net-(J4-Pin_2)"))
 (segment (start 98.815 106.04) (end 98.815 110.475) (width 1) (layer "F.Cu") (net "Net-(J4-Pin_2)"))
 (segment (start 98.815 110.475) (end 98.84 110.5) (width 1) (layer "F.Cu") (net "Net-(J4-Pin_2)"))
 (segment (start 55.315 102.54) (end 55.315 106.975) (width 1) (layer "F.Cu") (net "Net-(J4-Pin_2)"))
 (segment (start 50.84 100.29) (end 50.84 104.5) (width 1) (layer "F.Cu") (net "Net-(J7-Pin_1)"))
 (segment (start 94.34 103.79) (end 94.34 108) (width 1) (layer "F.Cu") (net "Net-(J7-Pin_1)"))
 (segment (start 91.09 79.125) (end 96.235 79.125) (width 1) (layer "F.Cu") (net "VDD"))
 (segment (start 47.59 75.625) (end 52.735 75.625) (width 1) (layer "F.Cu") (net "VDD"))
 (segment (start 96.235 79.125) (end 96.25 79.11) (width 1) (layer "F.Cu") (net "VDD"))
 (segment (start 52.735 75.625) (end 52.75 75.61) (width 1) (layer "F.Cu") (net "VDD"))
 (segment (start 47.59 78.165) (end 52.735 78.165) (width 1) (layer "F.Cu") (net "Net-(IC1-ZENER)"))
 (segment (start 91.09 81.665) (end 96.235 81.665) (width 1) (layer "F.Cu") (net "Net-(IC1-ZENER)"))
 (segment (start 52.735 78.165) (end 52.75 78.15) (width 1) (layer "F.Cu") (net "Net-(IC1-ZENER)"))
 (segment (start 96.235 81.665) (end 96.25 81.65) (width 1) (layer "F.Cu") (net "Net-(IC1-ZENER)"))
 (segment (start 96.235 84.205) (end 96.25 84.19) (width 1) (layer "F.Cu") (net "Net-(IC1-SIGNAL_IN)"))
 (segment (start 91.09 84.205) (end 96.235 84.205) (width 1) (layer "F.Cu") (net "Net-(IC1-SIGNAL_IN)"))
 (segment (start 52.735 80.705) (end 52.75 80.69) (width 1) (layer "F.Cu") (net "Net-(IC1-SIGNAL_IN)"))
 (segment (start 47.59 80.705) (end 52.735 80.705) (width 1) (layer "F.Cu") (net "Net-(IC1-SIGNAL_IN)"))
 (segment (start 43.025 97.75) (end 43.025 95.54) (width 1) (layer "F.Cu") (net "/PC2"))
 (segment (start 87.565 98) (end 87.565 89) (width 1) (layer "F.Cu") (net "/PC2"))
 (segment (start 46.32 83.245) (end 47.59 83.245) (width 1) (layer "F.Cu") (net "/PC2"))
 (segment (start 47.59 83.245) (end 52.735 83.245) (width 1) (layer "F.Cu") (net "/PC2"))
 (segment (start 89.82 86.745) (end 91.09 86.745) (width 1) (layer "F.Cu") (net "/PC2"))
 (segment (start 86.525 101.25) (end 86.525 99.04) (width 1) (layer "F.Cu") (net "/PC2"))
 (segment (start 44.065 85.5) (end 46.32 83.245) (width 1) (layer "F.Cu") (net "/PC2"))
 (segment (start 87.565 89) (end 89.82 86.745) (width 1) (layer "F.Cu") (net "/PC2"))
 (segment (start 52.735 83.245) (end 52.75 83.23) (width 1) (layer "F.Cu") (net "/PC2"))
 (segment (start 91.09 86.745) (end 96.235 86.745) (width 1) (layer "F.Cu") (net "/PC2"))
 (segment (start 43.025 95.54) (end 44.065 94.5) (width 1) (layer "F.Cu") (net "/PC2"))
 (segment (start 86.525 99.04) (end 87.565 98) (width 1) (layer "F.Cu") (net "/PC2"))
 (segment (start 96.235 86.745) (end 96.25 86.73) (width 1) (layer "F.Cu") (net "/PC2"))
 (segment (start 44.065 94.5) (end 44.065 85.5) (width 1) (layer "F.Cu") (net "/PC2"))
 (segment (start 47.59 85.785) (end 52.735 85.785) (width 1) (layer "F.Cu") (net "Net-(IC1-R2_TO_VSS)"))
 (segment (start 96.235 89.285) (end 96.25 89.27) (width 1) (layer "F.Cu") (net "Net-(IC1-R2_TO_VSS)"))
 (segment (start 52.735 85.785) (end 52.75 85.77) (width 1) (layer "F.Cu") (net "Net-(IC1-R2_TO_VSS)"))
 (segment (start 91.09 89.285) (end 96.235 89.285) (width 1) (layer "F.Cu") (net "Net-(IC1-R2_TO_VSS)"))
 (segment (start 47.59 88.325) (end 52.735 88.325) (width 1) (layer "F.Cu") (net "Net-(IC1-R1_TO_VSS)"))
 (segment (start 96.235 91.825) (end 96.25 91.81) (width 1) (layer "F.Cu") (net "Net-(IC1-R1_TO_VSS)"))
 (segment (start 52.735 88.325) (end 52.75 88.31) (width 1) (layer "F.Cu") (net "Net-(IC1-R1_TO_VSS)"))
 (segment (start 91.09 91.825) (end 96.235 91.825) (width 1) (layer "F.Cu") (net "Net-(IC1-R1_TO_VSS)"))
 (segment (start 96.235 94.365) (end 96.25 94.35) (width 1) (layer "F.Cu") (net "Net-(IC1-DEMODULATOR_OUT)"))
 (segment (start 47.59 90.865) (end 52.735 90.865) (width 1) (layer "F.Cu") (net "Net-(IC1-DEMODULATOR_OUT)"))
 (segment (start 91.09 94.365) (end 96.235 94.365) (width 1) (layer "F.Cu") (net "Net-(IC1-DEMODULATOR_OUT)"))
 (segment (start 52.735 90.865) (end 52.75 90.85) (width 1) (layer "F.Cu") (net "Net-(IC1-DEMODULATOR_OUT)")))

